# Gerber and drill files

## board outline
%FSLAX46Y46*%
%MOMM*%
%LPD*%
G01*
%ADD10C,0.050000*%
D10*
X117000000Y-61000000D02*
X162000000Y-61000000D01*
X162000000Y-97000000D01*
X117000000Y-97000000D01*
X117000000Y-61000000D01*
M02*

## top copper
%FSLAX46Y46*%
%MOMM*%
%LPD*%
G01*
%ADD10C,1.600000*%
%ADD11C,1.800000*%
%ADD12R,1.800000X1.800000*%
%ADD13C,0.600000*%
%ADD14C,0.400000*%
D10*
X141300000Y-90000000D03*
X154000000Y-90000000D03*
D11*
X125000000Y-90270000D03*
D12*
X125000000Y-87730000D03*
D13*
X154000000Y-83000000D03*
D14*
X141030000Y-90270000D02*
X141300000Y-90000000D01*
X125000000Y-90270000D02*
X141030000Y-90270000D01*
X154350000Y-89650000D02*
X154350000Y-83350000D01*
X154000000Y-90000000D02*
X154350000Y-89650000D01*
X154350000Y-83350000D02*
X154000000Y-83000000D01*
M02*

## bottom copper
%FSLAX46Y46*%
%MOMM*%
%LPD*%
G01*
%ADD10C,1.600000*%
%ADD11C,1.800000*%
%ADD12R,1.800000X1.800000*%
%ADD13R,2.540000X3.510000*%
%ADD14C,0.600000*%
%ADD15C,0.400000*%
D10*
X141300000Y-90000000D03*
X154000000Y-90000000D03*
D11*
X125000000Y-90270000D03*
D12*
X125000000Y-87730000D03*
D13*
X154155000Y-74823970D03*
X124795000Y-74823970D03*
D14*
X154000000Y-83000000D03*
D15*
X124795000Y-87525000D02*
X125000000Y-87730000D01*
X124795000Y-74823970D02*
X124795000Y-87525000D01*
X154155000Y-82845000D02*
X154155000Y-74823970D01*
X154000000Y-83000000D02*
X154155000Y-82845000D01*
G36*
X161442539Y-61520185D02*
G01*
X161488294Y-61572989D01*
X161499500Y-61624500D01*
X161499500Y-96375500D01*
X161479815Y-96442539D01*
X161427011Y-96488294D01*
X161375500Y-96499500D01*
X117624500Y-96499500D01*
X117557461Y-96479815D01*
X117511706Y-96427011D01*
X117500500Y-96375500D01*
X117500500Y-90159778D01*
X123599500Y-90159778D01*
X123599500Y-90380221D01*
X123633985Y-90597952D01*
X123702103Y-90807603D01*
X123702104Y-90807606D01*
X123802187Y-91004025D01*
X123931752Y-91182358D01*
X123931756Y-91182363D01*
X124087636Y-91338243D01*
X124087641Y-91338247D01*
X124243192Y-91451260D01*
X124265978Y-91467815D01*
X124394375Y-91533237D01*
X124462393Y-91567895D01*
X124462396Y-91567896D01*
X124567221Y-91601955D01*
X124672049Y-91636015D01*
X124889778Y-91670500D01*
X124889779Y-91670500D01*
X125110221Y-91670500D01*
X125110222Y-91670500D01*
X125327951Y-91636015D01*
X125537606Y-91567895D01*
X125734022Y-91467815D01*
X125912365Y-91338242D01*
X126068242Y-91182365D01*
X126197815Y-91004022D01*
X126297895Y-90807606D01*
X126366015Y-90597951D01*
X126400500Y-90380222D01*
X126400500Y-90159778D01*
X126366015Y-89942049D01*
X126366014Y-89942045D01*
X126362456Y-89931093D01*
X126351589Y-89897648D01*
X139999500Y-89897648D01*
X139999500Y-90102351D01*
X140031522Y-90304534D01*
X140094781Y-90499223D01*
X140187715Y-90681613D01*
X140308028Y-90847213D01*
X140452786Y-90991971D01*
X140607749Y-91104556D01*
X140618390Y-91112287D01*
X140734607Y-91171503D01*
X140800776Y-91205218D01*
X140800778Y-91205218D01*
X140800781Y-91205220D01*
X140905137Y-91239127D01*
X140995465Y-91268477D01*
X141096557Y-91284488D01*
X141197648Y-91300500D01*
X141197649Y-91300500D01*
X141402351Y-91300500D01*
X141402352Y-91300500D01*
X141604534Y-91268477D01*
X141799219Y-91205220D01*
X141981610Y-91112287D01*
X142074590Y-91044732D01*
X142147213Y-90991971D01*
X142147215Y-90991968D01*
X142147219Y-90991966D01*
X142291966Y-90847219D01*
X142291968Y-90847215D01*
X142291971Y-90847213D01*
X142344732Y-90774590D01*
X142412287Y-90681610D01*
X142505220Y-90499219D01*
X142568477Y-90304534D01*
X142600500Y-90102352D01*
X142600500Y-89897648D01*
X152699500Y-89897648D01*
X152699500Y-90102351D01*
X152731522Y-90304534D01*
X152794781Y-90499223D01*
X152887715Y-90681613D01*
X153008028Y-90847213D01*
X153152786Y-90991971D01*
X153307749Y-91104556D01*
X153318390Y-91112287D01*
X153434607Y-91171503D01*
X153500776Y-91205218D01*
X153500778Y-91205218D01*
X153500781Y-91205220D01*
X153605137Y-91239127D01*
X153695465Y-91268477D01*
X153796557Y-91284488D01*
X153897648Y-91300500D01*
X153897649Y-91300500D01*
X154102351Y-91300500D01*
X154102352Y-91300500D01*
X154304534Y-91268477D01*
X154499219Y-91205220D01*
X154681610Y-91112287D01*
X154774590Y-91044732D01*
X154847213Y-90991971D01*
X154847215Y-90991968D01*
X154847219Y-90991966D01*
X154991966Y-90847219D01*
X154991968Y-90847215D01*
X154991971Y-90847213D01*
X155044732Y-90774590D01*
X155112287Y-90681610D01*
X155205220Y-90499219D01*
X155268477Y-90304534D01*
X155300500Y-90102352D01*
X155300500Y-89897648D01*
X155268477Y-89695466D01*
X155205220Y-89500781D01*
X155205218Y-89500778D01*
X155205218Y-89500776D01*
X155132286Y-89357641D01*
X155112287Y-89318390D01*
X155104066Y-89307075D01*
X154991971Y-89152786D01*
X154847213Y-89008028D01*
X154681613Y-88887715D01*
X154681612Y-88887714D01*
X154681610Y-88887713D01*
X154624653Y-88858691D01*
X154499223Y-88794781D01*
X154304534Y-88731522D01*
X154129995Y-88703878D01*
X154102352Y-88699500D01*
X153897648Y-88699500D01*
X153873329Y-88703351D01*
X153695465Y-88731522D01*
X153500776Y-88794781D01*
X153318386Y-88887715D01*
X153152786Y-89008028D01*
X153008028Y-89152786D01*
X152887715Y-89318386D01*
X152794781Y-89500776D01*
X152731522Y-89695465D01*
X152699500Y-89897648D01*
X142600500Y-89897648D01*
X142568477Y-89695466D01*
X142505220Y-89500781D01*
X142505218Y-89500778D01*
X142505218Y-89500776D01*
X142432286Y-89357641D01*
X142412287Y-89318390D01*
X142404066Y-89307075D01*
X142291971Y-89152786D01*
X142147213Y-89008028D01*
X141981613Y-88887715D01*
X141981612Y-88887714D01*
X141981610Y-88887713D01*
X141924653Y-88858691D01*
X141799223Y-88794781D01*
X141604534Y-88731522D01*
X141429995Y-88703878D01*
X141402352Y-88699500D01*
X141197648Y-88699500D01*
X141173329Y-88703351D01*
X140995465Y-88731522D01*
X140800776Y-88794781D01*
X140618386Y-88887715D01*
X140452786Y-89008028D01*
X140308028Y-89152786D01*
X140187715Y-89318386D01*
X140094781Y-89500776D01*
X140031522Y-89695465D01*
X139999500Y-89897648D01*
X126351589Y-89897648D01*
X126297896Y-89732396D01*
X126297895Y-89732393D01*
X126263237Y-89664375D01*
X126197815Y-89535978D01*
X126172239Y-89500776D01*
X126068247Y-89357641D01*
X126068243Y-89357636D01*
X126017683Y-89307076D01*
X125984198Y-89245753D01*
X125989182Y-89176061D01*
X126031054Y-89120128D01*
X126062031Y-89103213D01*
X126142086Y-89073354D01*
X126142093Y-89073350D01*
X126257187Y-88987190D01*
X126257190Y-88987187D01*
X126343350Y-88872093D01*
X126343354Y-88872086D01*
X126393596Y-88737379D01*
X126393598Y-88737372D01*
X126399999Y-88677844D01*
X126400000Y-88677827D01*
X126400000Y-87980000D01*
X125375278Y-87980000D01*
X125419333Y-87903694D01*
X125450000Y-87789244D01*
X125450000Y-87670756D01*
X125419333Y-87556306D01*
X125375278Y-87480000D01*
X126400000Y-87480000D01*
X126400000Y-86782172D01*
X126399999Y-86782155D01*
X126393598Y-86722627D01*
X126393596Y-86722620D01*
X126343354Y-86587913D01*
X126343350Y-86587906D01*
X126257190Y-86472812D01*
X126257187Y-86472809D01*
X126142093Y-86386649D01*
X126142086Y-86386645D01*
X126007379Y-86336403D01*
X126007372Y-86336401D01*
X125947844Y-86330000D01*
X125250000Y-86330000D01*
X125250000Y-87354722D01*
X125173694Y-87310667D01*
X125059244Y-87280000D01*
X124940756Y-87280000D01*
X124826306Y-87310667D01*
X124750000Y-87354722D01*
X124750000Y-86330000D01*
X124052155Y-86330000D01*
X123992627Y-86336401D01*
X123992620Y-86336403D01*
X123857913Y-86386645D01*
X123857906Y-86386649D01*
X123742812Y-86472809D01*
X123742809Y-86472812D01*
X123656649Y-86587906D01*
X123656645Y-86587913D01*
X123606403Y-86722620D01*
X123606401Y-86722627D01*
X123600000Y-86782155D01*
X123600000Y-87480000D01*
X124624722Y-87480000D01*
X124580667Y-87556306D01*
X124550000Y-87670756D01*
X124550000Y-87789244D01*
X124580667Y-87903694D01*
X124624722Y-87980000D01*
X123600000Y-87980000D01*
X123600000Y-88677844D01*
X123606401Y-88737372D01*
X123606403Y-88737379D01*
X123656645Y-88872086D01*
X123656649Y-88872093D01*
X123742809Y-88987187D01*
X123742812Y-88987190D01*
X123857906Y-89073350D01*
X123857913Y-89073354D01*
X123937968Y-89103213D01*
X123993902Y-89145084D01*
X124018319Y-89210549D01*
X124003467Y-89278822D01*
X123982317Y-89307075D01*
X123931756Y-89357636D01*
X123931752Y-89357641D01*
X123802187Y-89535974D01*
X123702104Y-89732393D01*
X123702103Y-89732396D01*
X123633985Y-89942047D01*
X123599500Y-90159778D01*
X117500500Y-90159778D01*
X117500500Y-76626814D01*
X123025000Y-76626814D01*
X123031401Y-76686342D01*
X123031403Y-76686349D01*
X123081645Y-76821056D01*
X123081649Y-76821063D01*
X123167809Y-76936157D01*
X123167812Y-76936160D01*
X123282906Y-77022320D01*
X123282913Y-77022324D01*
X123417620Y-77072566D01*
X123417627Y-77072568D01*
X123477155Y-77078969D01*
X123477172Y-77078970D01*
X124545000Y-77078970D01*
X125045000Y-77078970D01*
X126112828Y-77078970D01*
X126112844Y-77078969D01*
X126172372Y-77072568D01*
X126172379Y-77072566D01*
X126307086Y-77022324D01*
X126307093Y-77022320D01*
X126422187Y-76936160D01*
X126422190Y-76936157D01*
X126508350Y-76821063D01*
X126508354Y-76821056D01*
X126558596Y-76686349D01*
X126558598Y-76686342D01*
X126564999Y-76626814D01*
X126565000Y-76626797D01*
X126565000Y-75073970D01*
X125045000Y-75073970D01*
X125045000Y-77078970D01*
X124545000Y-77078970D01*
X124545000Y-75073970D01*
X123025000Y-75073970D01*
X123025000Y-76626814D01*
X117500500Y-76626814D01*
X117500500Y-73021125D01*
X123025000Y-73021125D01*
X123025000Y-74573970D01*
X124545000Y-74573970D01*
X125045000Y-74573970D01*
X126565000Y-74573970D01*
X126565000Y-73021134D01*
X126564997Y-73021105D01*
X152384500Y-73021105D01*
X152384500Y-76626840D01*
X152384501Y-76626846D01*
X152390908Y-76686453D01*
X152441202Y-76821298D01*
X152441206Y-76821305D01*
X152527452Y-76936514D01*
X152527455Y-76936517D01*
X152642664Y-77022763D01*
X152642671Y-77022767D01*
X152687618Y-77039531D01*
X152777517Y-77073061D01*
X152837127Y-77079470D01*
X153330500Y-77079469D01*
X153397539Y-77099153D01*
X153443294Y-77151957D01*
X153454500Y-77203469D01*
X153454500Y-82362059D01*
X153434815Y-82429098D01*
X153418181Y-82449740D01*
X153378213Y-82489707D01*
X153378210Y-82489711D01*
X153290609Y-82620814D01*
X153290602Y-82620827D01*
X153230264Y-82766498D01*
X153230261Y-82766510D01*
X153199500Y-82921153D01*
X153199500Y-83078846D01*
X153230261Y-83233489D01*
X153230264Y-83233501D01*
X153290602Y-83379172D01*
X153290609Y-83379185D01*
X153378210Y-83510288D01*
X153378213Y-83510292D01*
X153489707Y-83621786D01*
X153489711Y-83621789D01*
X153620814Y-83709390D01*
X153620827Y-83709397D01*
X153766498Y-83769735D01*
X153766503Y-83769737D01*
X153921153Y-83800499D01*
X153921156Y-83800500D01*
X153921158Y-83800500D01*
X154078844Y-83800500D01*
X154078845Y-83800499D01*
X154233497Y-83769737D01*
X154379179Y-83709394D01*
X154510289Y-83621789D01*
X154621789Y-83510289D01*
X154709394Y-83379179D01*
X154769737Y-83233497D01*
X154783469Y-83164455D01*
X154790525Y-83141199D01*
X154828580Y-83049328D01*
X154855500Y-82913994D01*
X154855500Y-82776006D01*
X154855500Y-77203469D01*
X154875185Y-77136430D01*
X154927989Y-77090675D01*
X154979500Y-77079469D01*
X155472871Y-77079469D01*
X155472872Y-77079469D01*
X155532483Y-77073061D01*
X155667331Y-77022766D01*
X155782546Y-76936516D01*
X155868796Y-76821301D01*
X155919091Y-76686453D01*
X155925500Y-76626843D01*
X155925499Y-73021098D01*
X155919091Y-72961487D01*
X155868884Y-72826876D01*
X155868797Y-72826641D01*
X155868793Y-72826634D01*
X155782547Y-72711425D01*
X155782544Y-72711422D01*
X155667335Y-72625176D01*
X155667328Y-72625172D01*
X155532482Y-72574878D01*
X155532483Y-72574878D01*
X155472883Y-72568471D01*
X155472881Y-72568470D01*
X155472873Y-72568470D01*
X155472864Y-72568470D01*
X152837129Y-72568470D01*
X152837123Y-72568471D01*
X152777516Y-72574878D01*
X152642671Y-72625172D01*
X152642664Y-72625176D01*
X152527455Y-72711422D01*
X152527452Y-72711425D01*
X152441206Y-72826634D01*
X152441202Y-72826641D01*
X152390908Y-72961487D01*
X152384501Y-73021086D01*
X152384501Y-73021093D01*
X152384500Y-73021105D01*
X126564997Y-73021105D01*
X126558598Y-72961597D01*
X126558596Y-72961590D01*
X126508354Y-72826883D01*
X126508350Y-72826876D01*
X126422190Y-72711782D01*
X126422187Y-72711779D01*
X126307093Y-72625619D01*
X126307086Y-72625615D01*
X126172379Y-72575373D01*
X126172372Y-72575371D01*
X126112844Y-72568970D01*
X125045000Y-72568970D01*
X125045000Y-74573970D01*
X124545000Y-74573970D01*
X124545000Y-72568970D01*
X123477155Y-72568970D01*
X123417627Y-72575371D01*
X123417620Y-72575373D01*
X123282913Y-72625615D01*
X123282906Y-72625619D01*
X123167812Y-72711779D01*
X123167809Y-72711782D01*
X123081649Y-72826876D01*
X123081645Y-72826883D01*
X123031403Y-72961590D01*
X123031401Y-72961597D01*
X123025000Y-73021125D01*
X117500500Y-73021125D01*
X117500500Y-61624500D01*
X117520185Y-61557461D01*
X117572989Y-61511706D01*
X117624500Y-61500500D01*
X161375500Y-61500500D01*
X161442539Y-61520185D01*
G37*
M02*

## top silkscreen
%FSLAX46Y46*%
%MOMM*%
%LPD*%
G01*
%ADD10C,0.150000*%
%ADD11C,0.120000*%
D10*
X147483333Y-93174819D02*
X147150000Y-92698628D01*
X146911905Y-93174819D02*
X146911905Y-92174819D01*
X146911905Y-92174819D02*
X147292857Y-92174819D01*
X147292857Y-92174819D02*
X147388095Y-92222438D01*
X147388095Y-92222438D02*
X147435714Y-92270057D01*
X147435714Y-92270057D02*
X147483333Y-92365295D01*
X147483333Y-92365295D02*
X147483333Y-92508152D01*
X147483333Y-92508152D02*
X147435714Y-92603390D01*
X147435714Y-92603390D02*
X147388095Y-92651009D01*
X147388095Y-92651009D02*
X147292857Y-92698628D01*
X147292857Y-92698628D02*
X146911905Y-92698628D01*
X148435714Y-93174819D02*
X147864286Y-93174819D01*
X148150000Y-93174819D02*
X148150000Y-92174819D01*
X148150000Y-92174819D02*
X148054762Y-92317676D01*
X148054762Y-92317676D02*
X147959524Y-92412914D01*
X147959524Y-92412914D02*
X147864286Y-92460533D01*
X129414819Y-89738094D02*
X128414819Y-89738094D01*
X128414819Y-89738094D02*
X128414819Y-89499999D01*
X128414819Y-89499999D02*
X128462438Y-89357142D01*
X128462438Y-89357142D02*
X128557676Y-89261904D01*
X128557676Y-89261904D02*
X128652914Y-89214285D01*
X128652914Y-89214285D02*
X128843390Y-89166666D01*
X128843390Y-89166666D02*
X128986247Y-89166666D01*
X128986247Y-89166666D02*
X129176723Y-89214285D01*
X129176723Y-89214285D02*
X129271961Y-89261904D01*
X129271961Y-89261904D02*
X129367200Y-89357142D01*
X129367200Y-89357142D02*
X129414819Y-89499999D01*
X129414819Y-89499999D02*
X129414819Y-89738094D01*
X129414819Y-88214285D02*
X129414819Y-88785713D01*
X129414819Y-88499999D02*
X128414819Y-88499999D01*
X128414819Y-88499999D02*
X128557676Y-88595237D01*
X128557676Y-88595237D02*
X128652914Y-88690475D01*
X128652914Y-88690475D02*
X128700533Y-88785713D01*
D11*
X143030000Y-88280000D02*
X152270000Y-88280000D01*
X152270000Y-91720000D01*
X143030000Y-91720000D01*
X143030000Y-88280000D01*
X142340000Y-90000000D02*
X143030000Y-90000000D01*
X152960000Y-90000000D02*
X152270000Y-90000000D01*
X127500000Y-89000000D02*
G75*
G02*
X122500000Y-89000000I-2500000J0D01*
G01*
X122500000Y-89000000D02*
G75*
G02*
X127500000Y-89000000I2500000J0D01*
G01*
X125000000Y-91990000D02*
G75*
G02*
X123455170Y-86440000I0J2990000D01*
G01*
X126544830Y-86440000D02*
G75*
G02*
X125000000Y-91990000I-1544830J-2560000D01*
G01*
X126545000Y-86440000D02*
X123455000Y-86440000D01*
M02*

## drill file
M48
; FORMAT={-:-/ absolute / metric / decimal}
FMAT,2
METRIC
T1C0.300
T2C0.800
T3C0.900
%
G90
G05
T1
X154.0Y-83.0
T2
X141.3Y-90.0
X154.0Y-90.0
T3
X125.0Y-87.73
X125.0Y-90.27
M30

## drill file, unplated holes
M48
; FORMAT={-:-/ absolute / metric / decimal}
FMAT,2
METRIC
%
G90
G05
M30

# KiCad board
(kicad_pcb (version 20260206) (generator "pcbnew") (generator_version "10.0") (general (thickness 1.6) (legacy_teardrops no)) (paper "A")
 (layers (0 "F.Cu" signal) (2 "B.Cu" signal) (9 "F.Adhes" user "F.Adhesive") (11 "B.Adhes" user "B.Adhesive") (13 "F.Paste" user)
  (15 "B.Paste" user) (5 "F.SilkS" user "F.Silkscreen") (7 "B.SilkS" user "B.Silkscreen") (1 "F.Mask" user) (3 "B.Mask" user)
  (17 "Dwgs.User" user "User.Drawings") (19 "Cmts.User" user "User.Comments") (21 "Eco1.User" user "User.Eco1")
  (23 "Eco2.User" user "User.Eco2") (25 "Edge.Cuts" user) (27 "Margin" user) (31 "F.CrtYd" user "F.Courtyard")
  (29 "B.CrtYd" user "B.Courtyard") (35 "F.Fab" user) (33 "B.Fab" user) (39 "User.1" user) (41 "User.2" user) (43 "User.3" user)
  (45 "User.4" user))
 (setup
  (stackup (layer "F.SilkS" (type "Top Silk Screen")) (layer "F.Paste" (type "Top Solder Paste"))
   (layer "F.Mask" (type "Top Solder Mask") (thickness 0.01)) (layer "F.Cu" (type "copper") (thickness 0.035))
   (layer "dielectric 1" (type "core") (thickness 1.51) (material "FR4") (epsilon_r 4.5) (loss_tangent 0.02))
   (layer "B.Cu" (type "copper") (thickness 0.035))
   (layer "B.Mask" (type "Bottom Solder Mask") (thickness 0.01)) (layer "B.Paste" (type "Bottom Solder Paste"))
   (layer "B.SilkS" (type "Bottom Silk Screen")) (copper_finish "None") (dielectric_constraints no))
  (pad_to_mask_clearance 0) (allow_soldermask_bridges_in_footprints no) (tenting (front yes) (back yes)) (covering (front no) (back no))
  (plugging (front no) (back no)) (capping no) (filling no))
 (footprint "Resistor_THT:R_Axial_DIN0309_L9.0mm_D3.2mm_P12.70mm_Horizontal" (layer "F.Cu") (at 154 90 180)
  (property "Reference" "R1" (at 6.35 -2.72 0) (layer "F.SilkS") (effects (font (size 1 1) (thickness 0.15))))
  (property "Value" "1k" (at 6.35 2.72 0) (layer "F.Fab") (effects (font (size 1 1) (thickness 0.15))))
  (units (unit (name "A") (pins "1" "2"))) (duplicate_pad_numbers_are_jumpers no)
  (fp_line (start 11.66 0) (end 10.97 0) (stroke (width 0.12) (type solid)) (layer "F.SilkS"))
  (fp_line (start 1.04 0) (end 1.73 0) (stroke (width 0.12) (type solid)) (layer "F.SilkS"))
  (fp_rect (start 1.73 -1.72) (end 10.97 1.72) (stroke (width 0.12) (type solid)) (fill no) (layer "F.SilkS"))
  (pad "1" thru_hole circle (at 0 0 180) (size 1.6 1.6) (drill 0.8) (layers "*.Cu" "*.Mask") (remove_unused_layers no) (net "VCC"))
  (pad "2" thru_hole circle (at 12.7 0 180) (size 1.6 1.6) (drill 0.8) (layers "*.Cu" "*.Mask") (remove_unused_layers no) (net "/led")))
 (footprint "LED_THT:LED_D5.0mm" (layer "F.Cu") (at 125 87.73 -90)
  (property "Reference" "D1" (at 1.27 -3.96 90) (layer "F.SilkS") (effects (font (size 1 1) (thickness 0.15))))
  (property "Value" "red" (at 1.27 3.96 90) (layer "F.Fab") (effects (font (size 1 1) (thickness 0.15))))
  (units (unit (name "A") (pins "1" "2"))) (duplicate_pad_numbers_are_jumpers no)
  (fp_line (start -1.29 -1.545) (end -1.29 1.545) (stroke (width 0.12) (type solid)) (layer "F.SilkS"))
  (fp_arc (start 4.26 0) (mid 2.071779 2.880495) (end -1.29 1.54483) (stroke (width 0.12) (type solid)) (layer "F.SilkS"))
  (fp_arc (start -1.29 -1.54483) (mid 2.071779 -2.880495) (end 4.26 0) (stroke (width 0.12) (type solid)) (layer "F.SilkS"))
  (fp_circle (center 1.27 0) (end 3.77 0) (stroke (width 0.12) (type solid)) (fill no) (layer "F.SilkS"))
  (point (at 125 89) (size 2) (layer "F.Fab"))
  (pad "1" thru_hole rect (at 0 0 270) (size 1.8 1.8) (drill 0.9) (layers "*.Cu" "*.Mask") (remove_unused_layers no) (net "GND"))
  (pad "2" thru_hole circle (at 2.54 0 270) (size 1.8 1.8) (drill 0.9) (layers "*.Cu" "*.Mask") (remove_unused_layers no) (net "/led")))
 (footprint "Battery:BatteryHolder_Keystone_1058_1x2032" (layer "B.Cu") (at 139.475 74.82397 180)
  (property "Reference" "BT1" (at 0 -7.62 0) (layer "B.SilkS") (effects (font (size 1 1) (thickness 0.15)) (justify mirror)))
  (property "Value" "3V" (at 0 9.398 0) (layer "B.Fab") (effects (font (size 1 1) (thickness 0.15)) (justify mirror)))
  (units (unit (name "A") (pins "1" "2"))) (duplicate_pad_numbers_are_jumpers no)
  (pad "1" smd rect (at -14.68 0 180) (size 2.54 3.51) (layers "B.Cu" "B.Mask" "B.Paste") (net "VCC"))
  (pad "2" smd rect (at 14.68 0 180) (size 2.54 3.51) (layers "B.Cu" "B.Mask" "B.Paste") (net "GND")))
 (gr_rect (start 117 61) (end 162 97) (stroke (width 0.05) (type default)) (fill no) (layer "Edge.Cuts"))
 (segment (start 154 90) (end 154.35 89.65) (width 0.4) (layer "F.Cu") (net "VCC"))
 (segment (start 154.35 83.35) (end 154 83) (width 0.4) (layer "F.Cu") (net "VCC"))
 (segment (start 154.35 89.65) (end 154.35 83.35) (width 0.4) (layer "F.Cu") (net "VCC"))
 (via (at 154 83) (size 0.6) (drill 0.3) (layers "F.Cu" "B.Cu") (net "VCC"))
 (segment (start 154 83) (end 154.155 82.845) (width 0.4) (layer "B.Cu") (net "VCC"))
 (segment (start 154.155 82.845) (end 154.155 74.82397) (width 0.4) (layer "B.Cu") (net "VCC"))
 (segment (start 141.03 90.27) (end 141.3 90) (width 0.4) (layer "F.Cu") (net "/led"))
 (segment (start 125 90.27) (end 141.03 90.27) (width 0.4) (layer "F.Cu") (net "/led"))
 (segment (start 124.795 87.525) (end 125 87.73) (width 0.4) (layer "B.Cu") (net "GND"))
 (segment (start 124.795 74.82397) (end 124.795 87.525) (width 0.4) (layer "B.Cu") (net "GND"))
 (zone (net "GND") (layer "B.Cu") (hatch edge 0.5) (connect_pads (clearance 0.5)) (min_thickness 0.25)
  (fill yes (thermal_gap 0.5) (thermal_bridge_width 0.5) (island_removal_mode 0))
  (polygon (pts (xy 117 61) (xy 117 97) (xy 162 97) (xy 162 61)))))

